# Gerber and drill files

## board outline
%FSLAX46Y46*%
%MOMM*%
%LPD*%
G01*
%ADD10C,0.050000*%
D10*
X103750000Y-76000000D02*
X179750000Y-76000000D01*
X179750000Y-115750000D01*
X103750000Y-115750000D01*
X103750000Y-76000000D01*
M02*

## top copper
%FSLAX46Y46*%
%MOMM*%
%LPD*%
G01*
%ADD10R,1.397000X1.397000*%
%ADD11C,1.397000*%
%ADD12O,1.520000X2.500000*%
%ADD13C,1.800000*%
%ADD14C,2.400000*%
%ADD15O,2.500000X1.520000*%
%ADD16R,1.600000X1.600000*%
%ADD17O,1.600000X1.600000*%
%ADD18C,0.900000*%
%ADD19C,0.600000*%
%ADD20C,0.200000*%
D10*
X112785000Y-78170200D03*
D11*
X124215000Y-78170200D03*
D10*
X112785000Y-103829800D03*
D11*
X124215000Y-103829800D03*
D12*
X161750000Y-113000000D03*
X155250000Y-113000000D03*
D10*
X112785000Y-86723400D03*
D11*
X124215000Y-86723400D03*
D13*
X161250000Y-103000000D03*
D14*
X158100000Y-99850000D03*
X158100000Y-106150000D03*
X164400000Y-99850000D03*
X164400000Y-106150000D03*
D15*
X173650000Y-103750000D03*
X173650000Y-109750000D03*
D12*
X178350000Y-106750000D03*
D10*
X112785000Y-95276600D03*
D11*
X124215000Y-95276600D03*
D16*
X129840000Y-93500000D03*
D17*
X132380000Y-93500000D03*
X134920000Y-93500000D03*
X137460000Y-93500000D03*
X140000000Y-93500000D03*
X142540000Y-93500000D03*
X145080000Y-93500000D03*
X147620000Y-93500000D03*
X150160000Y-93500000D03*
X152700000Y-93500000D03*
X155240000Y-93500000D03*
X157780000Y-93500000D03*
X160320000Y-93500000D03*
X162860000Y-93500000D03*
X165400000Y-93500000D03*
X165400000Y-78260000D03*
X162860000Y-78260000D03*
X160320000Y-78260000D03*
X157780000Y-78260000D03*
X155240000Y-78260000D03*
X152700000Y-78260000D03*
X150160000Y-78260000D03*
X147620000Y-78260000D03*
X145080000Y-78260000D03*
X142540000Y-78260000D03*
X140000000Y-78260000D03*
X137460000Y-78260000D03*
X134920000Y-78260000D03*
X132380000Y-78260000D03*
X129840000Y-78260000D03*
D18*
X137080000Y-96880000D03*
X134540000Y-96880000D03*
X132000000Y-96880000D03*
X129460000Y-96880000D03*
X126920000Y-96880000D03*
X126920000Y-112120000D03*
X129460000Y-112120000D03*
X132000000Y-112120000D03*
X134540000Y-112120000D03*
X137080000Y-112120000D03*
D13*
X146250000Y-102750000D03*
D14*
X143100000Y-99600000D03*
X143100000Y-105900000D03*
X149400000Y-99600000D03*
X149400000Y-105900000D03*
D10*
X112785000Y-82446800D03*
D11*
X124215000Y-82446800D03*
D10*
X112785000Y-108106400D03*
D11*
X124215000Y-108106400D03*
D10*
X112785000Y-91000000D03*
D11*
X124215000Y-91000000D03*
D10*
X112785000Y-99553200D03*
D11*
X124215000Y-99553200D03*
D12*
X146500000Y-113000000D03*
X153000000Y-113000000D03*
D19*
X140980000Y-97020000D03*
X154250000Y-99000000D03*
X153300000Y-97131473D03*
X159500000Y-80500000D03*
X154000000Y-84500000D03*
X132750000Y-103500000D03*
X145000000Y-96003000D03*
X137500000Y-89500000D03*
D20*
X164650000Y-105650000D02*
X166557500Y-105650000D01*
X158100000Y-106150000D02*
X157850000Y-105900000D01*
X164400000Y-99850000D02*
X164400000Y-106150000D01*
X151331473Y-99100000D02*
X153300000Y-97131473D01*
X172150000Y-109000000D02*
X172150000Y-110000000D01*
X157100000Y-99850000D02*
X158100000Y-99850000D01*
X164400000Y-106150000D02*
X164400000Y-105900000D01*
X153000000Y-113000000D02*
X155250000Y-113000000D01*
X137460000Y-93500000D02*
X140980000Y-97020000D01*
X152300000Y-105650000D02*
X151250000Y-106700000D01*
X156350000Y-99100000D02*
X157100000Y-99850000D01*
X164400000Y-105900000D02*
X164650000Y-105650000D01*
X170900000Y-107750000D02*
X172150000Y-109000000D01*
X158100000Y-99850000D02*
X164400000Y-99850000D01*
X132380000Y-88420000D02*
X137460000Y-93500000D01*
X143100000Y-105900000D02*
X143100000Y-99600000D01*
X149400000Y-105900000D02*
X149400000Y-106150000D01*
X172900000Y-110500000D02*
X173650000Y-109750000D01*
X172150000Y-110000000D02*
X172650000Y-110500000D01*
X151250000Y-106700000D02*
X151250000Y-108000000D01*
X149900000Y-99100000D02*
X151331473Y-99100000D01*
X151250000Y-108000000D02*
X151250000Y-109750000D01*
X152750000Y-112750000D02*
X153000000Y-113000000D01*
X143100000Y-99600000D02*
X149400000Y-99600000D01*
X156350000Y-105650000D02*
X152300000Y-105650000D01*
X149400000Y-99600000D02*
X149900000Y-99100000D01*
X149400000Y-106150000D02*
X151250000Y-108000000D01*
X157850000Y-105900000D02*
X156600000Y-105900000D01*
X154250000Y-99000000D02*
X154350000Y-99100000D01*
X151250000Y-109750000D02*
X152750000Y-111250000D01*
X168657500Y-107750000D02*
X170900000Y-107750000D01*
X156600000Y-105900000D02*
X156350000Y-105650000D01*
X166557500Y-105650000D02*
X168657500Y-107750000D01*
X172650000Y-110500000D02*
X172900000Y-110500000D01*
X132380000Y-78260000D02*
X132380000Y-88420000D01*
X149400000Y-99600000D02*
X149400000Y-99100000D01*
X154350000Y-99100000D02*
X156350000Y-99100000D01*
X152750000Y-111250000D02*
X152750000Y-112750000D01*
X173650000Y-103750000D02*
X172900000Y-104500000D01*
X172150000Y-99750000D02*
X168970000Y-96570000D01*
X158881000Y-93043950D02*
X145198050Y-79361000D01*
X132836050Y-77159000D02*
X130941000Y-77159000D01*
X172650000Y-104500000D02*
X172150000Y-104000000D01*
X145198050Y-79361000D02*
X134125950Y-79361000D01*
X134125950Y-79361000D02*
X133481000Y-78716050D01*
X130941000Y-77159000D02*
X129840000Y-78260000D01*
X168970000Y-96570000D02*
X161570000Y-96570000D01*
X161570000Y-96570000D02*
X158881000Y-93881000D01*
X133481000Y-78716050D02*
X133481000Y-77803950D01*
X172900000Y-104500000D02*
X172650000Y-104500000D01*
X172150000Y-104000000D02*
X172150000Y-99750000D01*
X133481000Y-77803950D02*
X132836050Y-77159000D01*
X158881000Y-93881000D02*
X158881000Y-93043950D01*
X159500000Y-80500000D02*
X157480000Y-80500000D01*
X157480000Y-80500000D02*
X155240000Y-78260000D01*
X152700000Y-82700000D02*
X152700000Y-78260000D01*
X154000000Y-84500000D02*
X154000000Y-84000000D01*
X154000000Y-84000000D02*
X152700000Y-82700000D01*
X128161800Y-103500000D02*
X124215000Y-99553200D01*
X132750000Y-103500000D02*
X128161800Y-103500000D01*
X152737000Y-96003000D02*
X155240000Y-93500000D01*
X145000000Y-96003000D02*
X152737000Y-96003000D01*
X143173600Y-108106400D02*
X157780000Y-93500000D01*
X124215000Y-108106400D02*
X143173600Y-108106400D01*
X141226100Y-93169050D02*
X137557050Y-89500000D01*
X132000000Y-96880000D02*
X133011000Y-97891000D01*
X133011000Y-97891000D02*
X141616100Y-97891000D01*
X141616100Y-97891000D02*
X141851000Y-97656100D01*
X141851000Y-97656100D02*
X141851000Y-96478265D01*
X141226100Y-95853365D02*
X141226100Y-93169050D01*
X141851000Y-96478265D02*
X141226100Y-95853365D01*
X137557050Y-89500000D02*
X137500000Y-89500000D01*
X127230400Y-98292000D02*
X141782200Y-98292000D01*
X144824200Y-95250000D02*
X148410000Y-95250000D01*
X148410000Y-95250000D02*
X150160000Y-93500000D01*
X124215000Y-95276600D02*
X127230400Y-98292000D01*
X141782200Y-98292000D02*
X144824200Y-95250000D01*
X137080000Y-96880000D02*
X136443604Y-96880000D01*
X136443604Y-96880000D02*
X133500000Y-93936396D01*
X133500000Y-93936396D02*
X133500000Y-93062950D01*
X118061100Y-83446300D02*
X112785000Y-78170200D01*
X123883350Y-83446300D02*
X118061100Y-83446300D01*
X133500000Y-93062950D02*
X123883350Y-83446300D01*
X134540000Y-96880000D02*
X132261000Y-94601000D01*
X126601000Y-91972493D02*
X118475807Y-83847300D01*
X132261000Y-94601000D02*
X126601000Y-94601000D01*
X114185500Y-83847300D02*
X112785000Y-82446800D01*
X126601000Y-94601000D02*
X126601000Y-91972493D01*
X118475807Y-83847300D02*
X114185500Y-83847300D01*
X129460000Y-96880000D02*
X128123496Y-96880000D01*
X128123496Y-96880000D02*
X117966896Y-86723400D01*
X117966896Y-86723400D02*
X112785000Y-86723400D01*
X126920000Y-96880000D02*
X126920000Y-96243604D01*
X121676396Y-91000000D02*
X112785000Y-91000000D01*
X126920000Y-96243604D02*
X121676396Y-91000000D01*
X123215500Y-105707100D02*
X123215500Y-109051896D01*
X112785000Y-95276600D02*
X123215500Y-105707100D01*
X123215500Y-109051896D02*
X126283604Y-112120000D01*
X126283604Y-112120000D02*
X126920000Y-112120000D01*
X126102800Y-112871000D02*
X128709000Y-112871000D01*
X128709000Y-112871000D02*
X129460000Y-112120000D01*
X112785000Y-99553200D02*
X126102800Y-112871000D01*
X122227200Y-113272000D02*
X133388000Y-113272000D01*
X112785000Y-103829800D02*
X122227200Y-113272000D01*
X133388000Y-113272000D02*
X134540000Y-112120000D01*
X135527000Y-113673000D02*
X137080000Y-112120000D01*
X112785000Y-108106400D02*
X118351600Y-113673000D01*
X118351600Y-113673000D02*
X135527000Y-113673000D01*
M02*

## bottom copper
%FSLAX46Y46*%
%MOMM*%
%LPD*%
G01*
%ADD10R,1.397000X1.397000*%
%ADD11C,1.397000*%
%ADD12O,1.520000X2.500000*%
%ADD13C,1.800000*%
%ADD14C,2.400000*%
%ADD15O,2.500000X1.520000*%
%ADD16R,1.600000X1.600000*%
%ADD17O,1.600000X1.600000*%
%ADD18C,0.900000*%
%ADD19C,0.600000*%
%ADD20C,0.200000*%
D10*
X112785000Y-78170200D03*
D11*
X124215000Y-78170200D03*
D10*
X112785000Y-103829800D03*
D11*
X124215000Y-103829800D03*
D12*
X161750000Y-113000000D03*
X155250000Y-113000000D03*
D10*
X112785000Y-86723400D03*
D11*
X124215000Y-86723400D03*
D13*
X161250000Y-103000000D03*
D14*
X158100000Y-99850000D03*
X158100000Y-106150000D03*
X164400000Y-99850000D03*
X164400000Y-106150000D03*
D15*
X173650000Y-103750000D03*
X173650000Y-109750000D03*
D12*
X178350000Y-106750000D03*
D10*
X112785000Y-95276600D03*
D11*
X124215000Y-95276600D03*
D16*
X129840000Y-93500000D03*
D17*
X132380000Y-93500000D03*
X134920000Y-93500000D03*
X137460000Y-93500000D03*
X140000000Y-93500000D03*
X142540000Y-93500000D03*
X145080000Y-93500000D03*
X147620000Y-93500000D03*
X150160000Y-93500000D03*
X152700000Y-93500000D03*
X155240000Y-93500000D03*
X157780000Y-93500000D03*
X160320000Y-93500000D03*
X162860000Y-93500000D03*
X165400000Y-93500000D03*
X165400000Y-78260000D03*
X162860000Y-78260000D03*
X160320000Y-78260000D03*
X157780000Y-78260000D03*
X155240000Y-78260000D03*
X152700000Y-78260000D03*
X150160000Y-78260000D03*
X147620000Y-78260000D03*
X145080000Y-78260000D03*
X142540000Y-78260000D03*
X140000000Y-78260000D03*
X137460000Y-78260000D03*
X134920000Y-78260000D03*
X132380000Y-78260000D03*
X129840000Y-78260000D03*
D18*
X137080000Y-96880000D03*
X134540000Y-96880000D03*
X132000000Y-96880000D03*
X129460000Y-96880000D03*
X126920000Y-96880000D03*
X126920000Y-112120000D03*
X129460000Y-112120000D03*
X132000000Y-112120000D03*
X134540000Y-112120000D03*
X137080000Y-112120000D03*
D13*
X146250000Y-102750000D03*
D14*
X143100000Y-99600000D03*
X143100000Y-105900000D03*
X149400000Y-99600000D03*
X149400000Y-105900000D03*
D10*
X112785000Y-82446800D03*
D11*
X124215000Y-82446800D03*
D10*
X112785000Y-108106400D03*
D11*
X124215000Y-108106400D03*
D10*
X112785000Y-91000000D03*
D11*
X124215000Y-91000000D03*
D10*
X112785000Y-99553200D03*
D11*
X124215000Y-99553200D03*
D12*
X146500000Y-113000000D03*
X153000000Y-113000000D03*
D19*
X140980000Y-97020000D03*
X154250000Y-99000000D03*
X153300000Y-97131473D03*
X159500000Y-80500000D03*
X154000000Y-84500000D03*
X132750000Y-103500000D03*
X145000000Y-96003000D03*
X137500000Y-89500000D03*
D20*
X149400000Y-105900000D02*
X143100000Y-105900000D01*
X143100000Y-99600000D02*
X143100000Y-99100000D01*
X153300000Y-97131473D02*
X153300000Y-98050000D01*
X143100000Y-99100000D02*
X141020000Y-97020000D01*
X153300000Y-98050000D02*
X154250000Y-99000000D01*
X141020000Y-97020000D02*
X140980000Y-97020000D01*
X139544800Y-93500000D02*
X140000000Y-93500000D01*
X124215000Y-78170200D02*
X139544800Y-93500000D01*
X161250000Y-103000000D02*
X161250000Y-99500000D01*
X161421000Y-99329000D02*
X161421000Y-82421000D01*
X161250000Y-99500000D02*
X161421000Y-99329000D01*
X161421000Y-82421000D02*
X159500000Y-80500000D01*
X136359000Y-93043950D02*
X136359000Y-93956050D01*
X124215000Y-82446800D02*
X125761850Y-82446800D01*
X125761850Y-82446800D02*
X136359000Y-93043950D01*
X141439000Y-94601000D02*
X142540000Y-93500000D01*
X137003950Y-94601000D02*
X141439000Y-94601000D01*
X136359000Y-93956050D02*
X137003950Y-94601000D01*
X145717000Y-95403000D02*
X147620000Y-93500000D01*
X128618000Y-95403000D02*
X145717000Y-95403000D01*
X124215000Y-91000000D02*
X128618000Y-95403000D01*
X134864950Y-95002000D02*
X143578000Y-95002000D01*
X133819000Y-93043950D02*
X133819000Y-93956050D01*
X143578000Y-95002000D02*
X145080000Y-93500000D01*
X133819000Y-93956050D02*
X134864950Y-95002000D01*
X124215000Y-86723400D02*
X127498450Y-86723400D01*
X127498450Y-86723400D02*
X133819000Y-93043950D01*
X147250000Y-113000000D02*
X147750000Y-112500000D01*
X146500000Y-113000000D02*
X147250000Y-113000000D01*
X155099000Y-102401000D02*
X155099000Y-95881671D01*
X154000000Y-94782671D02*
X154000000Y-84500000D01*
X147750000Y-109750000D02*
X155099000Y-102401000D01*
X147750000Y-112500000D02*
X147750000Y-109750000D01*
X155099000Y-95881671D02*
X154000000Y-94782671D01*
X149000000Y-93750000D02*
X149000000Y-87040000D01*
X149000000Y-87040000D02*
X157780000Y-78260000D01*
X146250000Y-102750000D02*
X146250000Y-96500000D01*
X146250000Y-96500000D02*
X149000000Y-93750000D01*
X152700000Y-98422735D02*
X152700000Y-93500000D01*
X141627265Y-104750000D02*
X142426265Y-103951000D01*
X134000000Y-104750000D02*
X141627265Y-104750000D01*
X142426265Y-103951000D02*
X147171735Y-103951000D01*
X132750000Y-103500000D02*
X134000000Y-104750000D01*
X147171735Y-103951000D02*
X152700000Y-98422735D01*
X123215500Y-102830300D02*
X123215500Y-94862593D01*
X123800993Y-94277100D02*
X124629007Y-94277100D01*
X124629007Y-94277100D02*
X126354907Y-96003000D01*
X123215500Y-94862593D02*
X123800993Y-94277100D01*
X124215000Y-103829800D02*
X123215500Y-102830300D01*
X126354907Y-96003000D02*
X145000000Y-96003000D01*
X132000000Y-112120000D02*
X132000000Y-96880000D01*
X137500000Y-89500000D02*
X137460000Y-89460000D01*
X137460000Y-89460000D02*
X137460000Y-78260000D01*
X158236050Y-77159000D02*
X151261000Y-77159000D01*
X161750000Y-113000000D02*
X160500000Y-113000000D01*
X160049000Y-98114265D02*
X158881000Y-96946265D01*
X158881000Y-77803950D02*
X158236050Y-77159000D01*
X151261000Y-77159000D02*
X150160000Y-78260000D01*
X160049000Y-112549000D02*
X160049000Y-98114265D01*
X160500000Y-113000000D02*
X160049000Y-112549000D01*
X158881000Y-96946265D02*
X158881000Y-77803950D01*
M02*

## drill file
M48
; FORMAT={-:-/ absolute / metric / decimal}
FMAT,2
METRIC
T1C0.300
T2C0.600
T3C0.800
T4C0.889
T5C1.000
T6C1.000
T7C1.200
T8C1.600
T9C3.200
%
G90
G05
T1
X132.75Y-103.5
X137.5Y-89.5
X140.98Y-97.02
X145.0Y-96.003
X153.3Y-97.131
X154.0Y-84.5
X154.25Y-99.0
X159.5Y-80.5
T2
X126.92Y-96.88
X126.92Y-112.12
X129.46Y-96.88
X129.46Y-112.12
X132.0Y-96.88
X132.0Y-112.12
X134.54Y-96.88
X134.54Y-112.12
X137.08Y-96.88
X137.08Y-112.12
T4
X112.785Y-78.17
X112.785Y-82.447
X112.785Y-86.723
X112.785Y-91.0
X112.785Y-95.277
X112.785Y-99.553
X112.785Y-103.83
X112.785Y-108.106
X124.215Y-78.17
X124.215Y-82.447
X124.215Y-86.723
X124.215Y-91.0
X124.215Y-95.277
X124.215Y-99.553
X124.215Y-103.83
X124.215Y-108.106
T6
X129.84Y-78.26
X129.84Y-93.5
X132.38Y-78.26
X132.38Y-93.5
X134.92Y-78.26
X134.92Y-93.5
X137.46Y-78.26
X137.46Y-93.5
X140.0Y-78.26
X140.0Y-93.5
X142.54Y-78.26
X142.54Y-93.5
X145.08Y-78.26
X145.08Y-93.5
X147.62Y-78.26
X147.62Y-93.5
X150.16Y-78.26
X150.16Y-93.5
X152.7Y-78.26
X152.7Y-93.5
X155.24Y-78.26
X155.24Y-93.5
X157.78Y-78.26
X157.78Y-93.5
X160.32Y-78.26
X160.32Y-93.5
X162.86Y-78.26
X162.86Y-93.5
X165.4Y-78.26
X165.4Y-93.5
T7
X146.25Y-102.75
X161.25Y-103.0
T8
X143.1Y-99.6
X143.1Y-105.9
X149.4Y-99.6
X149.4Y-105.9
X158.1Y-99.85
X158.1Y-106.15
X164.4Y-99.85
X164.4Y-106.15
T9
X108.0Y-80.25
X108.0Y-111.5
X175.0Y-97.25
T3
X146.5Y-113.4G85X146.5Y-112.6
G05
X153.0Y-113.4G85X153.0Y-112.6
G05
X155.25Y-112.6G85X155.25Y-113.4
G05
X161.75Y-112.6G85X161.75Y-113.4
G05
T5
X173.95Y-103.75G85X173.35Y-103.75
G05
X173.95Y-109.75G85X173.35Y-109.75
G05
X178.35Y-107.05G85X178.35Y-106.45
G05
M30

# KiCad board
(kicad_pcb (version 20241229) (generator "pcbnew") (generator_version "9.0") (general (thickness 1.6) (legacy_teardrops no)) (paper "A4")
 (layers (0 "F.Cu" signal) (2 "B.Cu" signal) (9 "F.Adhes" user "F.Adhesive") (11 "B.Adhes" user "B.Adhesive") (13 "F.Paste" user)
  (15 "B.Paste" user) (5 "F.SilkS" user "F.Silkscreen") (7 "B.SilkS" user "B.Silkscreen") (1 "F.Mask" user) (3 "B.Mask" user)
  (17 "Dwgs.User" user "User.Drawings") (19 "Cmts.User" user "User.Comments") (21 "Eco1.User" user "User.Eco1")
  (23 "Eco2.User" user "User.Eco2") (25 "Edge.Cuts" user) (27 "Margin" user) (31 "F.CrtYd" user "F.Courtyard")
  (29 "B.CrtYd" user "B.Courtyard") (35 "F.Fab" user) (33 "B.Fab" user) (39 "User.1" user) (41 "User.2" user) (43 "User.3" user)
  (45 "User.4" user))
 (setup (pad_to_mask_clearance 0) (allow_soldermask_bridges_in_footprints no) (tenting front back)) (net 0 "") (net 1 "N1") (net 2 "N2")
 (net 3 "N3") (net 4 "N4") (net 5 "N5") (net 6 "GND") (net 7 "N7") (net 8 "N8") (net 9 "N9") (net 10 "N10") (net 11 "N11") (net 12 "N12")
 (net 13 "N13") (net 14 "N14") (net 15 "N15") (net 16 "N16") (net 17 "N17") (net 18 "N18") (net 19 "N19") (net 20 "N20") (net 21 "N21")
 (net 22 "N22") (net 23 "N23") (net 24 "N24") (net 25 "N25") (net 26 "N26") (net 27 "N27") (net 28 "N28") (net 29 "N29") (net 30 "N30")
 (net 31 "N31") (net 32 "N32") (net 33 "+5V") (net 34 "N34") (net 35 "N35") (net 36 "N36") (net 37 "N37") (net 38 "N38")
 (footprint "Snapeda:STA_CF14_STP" (layer "F.Cu") (at 112.785 78.1702)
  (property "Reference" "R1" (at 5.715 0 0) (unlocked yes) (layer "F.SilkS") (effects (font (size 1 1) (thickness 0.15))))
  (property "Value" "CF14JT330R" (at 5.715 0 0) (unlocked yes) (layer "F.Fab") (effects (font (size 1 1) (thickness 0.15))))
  (pad "1" thru_hole rect (at 0 0) (size 1.397 1.397) (drill 0.889) (layers "*.Cu" "*.Mask") (remove_unused_layers no) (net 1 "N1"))
  (pad "2" thru_hole circle (at 11.43 0) (size 1.397 1.397) (drill 0.889) (layers "*.Cu" "*.Mask") (remove_unused_layers no) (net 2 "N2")))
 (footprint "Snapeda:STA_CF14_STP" (layer "F.Cu") (at 112.785 103.8298)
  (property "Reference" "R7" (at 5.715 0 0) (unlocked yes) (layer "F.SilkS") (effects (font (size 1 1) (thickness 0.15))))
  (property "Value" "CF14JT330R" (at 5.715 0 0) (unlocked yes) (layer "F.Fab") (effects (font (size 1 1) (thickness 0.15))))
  (pad "1" thru_hole rect (at 0 0) (size 1.397 1.397) (drill 0.889) (layers "*.Cu" "*.Mask") (remove_unused_layers no) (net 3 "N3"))
  (pad "2" thru_hole circle (at 11.43 0) (size 1.397 1.397) (drill 0.889) (layers "*.Cu" "*.Mask") (remove_unused_layers no) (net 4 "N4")))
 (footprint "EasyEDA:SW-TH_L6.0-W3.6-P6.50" (layer "F.Cu") (at 158.5 113)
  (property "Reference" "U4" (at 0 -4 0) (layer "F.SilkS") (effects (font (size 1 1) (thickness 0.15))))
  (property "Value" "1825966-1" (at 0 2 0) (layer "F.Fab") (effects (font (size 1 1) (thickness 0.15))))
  (pad "1" thru_hole oval (at 3.25 0 270) (size 2.5 1.52) (drill oval 1.599997 0.799998) (layers "*.Cu" "*.Mask") (remove_unused_layers no)
   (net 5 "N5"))
  (pad "2" thru_hole oval (at -3.25 0 270) (size 2.5 1.52) (drill oval 1.599997 0.799998) (layers "*.Cu" "*.Mask") (remove_unused_layers no)
   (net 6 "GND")))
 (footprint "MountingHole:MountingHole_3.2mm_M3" (layer "F.Cu") (at 175 97.25)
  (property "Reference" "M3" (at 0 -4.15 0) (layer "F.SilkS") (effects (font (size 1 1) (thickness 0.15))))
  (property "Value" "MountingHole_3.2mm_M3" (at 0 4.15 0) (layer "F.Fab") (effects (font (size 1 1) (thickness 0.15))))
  (pad "" np_thru_hole circle (at 0 0) (size 3.2 3.2) (drill 3.2) (layers "*.Cu" "*.Mask")))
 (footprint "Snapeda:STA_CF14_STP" (layer "F.Cu") (at 112.785 86.7234)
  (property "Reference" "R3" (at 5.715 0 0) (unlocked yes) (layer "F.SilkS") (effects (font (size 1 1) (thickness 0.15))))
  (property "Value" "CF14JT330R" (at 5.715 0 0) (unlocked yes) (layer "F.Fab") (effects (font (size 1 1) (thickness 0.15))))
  (pad "1" thru_hole rect (at 0 0) (size 1.397 1.397) (drill 0.889) (layers "*.Cu" "*.Mask") (remove_unused_layers no) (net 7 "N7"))
  (pad "2" thru_hole circle (at 11.43 0) (size 1.397 1.397) (drill 0.889) (layers "*.Cu" "*.Mask") (remove_unused_layers no) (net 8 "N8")))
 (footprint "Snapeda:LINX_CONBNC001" (layer "F.Cu") (at 161.25 103)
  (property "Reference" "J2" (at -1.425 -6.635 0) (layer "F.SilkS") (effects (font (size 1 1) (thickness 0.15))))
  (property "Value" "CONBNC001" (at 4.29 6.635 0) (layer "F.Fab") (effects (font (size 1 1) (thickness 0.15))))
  (pad "1" thru_hole circle (at 0 0) (size 1.8 1.8) (drill 1.2) (layers "*.Cu" "*.Mask") (remove_unused_layers no) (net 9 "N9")
   (solder_mask_margin 0.102))
  (pad "S1" thru_hole circle (at -3.15 -3.15) (size 2.4 2.4) (drill 1.6) (layers "*.Cu" "*.Mask") (remove_unused_layers no) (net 6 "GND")
   (solder_mask_margin 0.102))
  (pad "S1" thru_hole circle (at -3.15 3.15) (size 2.4 2.4) (drill 1.6) (layers "*.Cu" "*.Mask") (remove_unused_layers no) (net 6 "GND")
   (solder_mask_margin 0.102))
  (pad "S1" thru_hole circle (at 3.15 -3.15) (size 2.4 2.4) (drill 1.6) (layers "*.Cu" "*.Mask") (remove_unused_layers no) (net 6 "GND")
   (solder_mask_margin 0.102))
  (pad "S1" thru_hole circle (at 3.15 3.15) (size 2.4 2.4) (drill 1.6) (layers "*.Cu" "*.Mask") (remove_unused_layers no) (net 6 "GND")
   (solder_mask_margin 0.102)))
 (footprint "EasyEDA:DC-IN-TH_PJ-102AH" (layer "F.Cu") (at 176 106.75 180)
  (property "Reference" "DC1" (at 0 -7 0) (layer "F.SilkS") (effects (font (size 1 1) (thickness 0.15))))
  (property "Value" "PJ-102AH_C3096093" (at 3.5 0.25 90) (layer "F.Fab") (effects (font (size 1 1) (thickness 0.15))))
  (pad "1" thru_hole oval (at 2.35 3 180) (size 2.5 1.52) (drill oval 1.599997 0.999998) (layers "*.Cu" "*.Mask") (remove_unused_layers no)
   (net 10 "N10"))
  (pad "2" thru_hole oval (at 2.35 -3 180) (size 2.5 1.52) (drill oval 1.599997 0.999998) (layers "*.Cu" "*.Mask") (remove_unused_layers no)
   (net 6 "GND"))
  (pad "3" thru_hole oval (at -2.35 0 90) (size 2.5 1.52) (drill oval 1.599997 0.999998) (layers "*.Cu" "*.Mask") (remove_unused_layers no)
   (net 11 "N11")))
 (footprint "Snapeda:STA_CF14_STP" (layer "F.Cu") (at 112.785 95.2766)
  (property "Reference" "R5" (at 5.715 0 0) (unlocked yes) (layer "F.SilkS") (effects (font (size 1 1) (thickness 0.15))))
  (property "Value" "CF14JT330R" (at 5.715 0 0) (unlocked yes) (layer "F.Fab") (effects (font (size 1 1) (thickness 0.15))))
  (pad "1" thru_hole rect (at 0 0) (size 1.397 1.397) (drill 0.889) (layers "*.Cu" "*.Mask") (remove_unused_layers no) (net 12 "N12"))
  (pad "2" thru_hole circle (at 11.43 0) (size 1.397 1.397) (drill 0.889) (layers "*.Cu" "*.Mask") (remove_unused_layers no) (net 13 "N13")))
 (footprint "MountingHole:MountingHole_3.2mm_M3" (layer "F.Cu") (at 108 111.5)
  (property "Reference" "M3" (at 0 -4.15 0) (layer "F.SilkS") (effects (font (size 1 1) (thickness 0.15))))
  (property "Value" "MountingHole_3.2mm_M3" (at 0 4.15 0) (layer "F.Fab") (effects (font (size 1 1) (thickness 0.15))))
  (pad "" np_thru_hole circle (at 0 0) (size 3.2 3.2) (drill 3.2) (layers "*.Cu" "*.Mask")))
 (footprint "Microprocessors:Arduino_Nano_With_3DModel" (layer "F.Cu") (at 129.84 93.5 90)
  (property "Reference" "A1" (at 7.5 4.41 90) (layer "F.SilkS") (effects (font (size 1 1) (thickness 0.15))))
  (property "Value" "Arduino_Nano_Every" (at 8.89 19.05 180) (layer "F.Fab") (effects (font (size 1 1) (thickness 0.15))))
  (pad "1" thru_hole rect (at 0 0 90) (size 1.6 1.6) (drill 1) (layers "*.Cu" "*.Mask") (remove_unused_layers no) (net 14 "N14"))
  (pad "2" thru_hole oval (at 0 2.54 90) (size 1.6 1.6) (drill 1) (layers "*.Cu" "*.Mask") (remove_unused_layers no) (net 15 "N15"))
  (pad "3" thru_hole oval (at 0 5.08 90) (size 1.6 1.6) (drill 1) (layers "*.Cu" "*.Mask") (remove_unused_layers no) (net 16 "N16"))
  (pad "4" thru_hole oval (at 0 7.62 90) (size 1.6 1.6) (drill 1) (layers "*.Cu" "*.Mask") (remove_unused_layers no) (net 6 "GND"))
  (pad "5" thru_hole oval (at 0 10.16 90) (size 1.6 1.6) (drill 1) (layers "*.Cu" "*.Mask") (remove_unused_layers no) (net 2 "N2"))
  (pad "6" thru_hole oval (at 0 12.7 90) (size 1.6 1.6) (drill 1) (layers "*.Cu" "*.Mask") (remove_unused_layers no) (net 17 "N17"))
  (pad "7" thru_hole oval (at 0 15.24 90) (size 1.6 1.6) (drill 1) (layers "*.Cu" "*.Mask") (remove_unused_layers no) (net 8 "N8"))
  (pad "8" thru_hole oval (at 0 17.78 90) (size 1.6 1.6) (drill 1) (layers "*.Cu" "*.Mask") (remove_unused_layers no) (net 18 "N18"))
  (pad "9" thru_hole oval (at 0 20.32 90) (size 1.6 1.6) (drill 1) (layers "*.Cu" "*.Mask") (remove_unused_layers no) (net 13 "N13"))
  (pad "10" thru_hole oval (at 0 22.86 90) (size 1.6 1.6) (drill 1) (layers "*.Cu" "*.Mask") (remove_unused_layers no) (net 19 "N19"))
  (pad "11" thru_hole oval (at 0 25.4 90) (size 1.6 1.6) (drill 1) (layers "*.Cu" "*.Mask") (remove_unused_layers no) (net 4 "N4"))
  (pad "12" thru_hole oval (at 0 27.94 90) (size 1.6 1.6) (drill 1) (layers "*.Cu" "*.Mask") (remove_unused_layers no) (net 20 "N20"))
  (pad "13" thru_hole oval (at 0 30.48 90) (size 1.6 1.6) (drill 1) (layers "*.Cu" "*.Mask") (remove_unused_layers no) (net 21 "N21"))
  (pad "14" thru_hole oval (at 0 33.02 90) (size 1.6 1.6) (drill 1) (layers "*.Cu" "*.Mask") (remove_unused_layers no) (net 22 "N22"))
  (pad "15" thru_hole oval (at 0 35.56 90) (size 1.6 1.6) (drill 1) (layers "*.Cu" "*.Mask") (remove_unused_layers no) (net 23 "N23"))
  (pad "16" thru_hole oval (at 15.24 35.56 90) (size 1.6 1.6) (drill 1) (layers "*.Cu" "*.Mask") (remove_unused_layers no) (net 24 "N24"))
  (pad "17" thru_hole oval (at 15.24 33.02 90) (size 1.6 1.6) (drill 1) (layers "*.Cu" "*.Mask") (remove_unused_layers no) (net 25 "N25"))
  (pad "18" thru_hole oval (at 15.24 30.48 90) (size 1.6 1.6) (drill 1) (layers "*.Cu" "*.Mask") (remove_unused_layers no) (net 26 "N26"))
  (pad "19" thru_hole oval (at 15.24 27.94 90) (size 1.6 1.6) (drill 1) (layers "*.Cu" "*.Mask") (remove_unused_layers no) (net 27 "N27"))
  (pad "20" thru_hole oval (at 15.24 25.4 90) (size 1.6 1.6) (drill 1) (layers "*.Cu" "*.Mask") (remove_unused_layers no) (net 9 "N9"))
  (pad "21" thru_hole oval (at 15.24 22.86 90) (size 1.6 1.6) (drill 1) (layers "*.Cu" "*.Mask") (remove_unused_layers no) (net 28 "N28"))
  (pad "22" thru_hole oval (at 15.24 20.32 90) (size 1.6 1.6) (drill 1) (layers "*.Cu" "*.Mask") (remove_unused_layers no) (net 5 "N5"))
  (pad "23" thru_hole oval (at 15.24 17.78 90) (size 1.6 1.6) (drill 1) (layers "*.Cu" "*.Mask") (remove_unused_layers no) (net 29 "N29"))
  (pad "24" thru_hole oval (at 15.24 15.24 90) (size 1.6 1.6) (drill 1) (layers "*.Cu" "*.Mask") (remove_unused_layers no) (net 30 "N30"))
  (pad "25" thru_hole oval (at 15.24 12.7 90) (size 1.6 1.6) (drill 1) (layers "*.Cu" "*.Mask") (remove_unused_layers no) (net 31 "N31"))
  (pad "26" thru_hole oval (at 15.24 10.16 90) (size 1.6 1.6) (drill 1) (layers "*.Cu" "*.Mask") (remove_unused_layers no) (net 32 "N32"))
  (pad "27" thru_hole oval (at 15.24 7.62 90) (size 1.6 1.6) (drill 1) (layers "*.Cu" "*.Mask") (remove_unused_layers no) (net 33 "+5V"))
  (pad "28" thru_hole oval (at 15.24 5.08 90) (size 1.6 1.6) (drill 1) (layers "*.Cu" "*.Mask") (remove_unused_layers no) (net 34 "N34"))
  (pad "29" thru_hole oval (at 15.24 2.54 90) (size 1.6 1.6) (drill 1) (layers "*.Cu" "*.Mask") (remove_unused_layers no) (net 6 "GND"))
  (pad "30" thru_hole oval (at 15.24 0 90) (size 1.6 1.6) (drill 1) (layers "*.Cu" "*.Mask") (remove_unused_layers no) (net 10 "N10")))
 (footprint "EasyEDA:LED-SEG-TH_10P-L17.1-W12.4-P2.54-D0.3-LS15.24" (layer "F.Cu") (at 132 104.5 180)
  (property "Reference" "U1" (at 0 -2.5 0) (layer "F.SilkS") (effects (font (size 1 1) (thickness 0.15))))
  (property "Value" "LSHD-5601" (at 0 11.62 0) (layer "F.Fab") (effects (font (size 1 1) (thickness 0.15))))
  (pad "1" thru_hole circle (at -5.08 7.62 180) (size 0.9 0.9) (drill 0.599999) (layers "*.Cu" "*.Mask") (remove_unused_layers no)
   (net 1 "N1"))
  (pad "2" thru_hole circle (at -2.54 7.62 180) (size 0.9 0.9) (drill 0.599999) (layers "*.Cu" "*.Mask") (remove_unused_layers no)
   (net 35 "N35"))
  (pad "3" thru_hole circle (at 0 7.62 180) (size 0.9 0.9) (drill 0.599999) (layers "*.Cu" "*.Mask") (remove_unused_layers no)
   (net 33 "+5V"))
  (pad "4" thru_hole circle (at 2.54 7.62 180) (size 0.9 0.9) (drill 0.599999) (layers "*.Cu" "*.Mask") (remove_unused_layers no)
   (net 7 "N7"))
  (pad "5" thru_hole circle (at 5.08 7.62 180) (size 0.9 0.9) (drill 0.599999) (layers "*.Cu" "*.Mask") (remove_unused_layers no)
   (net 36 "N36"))
  (pad "6" thru_hole circle (at 5.08 -7.62 180) (size 0.9 0.9) (drill 0.599999) (layers "*.Cu" "*.Mask") (remove_unused_layers no)
   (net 12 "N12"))
  (pad "7" thru_hole circle (at 2.54 -7.62 180) (size 0.9 0.9) (drill 0.599999) (layers "*.Cu" "*.Mask") (remove_unused_layers no)
   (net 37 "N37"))
  (pad "8" thru_hole circle (at 0 -7.62 180) (size 0.9 0.9) (drill 0.599999) (layers "*.Cu" "*.Mask") (remove_unused_layers no)
   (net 33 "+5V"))
  (pad "9" thru_hole circle (at -2.54 -7.62 180) (size 0.9 0.9) (drill 0.599999) (layers "*.Cu" "*.Mask") (remove_unused_layers no)
   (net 3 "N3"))
  (pad "10" thru_hole circle (at -5.08 -7.62 180) (size 0.9 0.9) (drill 0.599999) (layers "*.Cu" "*.Mask") (remove_unused_layers no)
   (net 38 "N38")))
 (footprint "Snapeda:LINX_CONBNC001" (layer "F.Cu") (at 146.25 102.75)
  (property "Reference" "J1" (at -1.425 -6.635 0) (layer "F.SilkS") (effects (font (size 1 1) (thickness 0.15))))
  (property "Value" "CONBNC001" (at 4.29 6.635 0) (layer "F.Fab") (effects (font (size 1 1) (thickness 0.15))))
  (pad "1" thru_hole circle (at 0 0) (size 1.8 1.8) (drill 1.2) (layers "*.Cu" "*.Mask") (remove_unused_layers no) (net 27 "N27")
   (solder_mask_margin 0.102))
  (pad "S1" thru_hole circle (at -3.15 -3.15) (size 2.4 2.4) (drill 1.6) (layers "*.Cu" "*.Mask") (remove_unused_layers no) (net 6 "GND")
   (solder_mask_margin 0.102))
  (pad "S1" thru_hole circle (at -3.15 3.15) (size 2.4 2.4) (drill 1.6) (layers "*.Cu" "*.Mask") (remove_unused_layers no) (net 6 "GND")
   (solder_mask_margin 0.102))
  (pad "S1" thru_hole circle (at 3.15 -3.15) (size 2.4 2.4) (drill 1.6) (layers "*.Cu" "*.Mask") (remove_unused_layers no) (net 6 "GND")
   (solder_mask_margin 0.102))
  (pad "S1" thru_hole circle (at 3.15 3.15) (size 2.4 2.4) (drill 1.6) (layers "*.Cu" "*.Mask") (remove_unused_layers no) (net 6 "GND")
   (solder_mask_margin 0.102)))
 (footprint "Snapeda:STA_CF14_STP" (layer "F.Cu") (at 112.785 82.4468)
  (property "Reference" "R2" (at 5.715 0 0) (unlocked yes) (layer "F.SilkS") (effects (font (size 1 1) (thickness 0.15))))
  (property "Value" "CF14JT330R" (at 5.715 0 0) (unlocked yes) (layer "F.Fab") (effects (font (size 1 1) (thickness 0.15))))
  (pad "1" thru_hole rect (at 0 0) (size 1.397 1.397) (drill 0.889) (layers "*.Cu" "*.Mask") (remove_unused_layers no) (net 35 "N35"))
  (pad "2" thru_hole circle (at 11.43 0) (size 1.397 1.397) (drill 0.889) (layers "*.Cu" "*.Mask") (remove_unused_layers no) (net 17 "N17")))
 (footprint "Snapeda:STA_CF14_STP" (layer "F.Cu") (at 112.785 108.1064)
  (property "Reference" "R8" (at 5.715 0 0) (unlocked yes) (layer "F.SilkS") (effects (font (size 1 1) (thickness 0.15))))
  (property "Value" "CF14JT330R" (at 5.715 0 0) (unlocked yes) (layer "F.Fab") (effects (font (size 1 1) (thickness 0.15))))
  (pad "1" thru_hole rect (at 0 0) (size 1.397 1.397) (drill 0.889) (layers "*.Cu" "*.Mask") (remove_unused_layers no) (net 38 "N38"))
  (pad "2" thru_hole circle (at 11.43 0) (size 1.397 1.397) (drill 0.889) (layers "*.Cu" "*.Mask") (remove_unused_layers no) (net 20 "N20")))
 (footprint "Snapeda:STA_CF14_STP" (layer "F.Cu") (at 112.785 91)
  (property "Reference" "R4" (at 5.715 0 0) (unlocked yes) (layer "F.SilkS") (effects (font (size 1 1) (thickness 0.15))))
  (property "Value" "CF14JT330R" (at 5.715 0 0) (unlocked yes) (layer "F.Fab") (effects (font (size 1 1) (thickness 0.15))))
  (pad "1" thru_hole rect (at 0 0) (size 1.397 1.397) (drill 0.889) (layers "*.Cu" "*.Mask") (remove_unused_layers no) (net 36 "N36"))
  (pad "2" thru_hole circle (at 11.43 0) (size 1.397 1.397) (drill 0.889) (layers "*.Cu" "*.Mask") (remove_unused_layers no) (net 18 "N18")))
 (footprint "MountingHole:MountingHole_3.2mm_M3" (layer "F.Cu") (at 108 80.25)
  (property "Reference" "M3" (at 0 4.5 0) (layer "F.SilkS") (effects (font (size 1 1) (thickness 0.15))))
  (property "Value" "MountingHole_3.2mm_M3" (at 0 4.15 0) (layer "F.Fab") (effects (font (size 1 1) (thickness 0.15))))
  (pad "" np_thru_hole circle (at 0 0) (size 3.2 3.2) (drill 3.2) (layers "*.Cu" "*.Mask")))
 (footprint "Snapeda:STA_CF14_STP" (layer "F.Cu") (at 112.785 99.5532)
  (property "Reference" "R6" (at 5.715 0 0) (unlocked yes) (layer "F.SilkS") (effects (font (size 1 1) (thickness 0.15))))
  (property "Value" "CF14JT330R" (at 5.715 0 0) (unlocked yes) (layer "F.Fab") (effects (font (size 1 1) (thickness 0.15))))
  (pad "1" thru_hole rect (at 0 0) (size 1.397 1.397) (drill 0.889) (layers "*.Cu" "*.Mask") (remove_unused_layers no) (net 37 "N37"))
  (pad "2" thru_hole circle (at 11.43 0) (size 1.397 1.397) (drill 0.889) (layers "*.Cu" "*.Mask") (remove_unused_layers no) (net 19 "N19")))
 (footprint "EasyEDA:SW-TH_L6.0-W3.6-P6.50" (layer "F.Cu") (at 149.75 113 180)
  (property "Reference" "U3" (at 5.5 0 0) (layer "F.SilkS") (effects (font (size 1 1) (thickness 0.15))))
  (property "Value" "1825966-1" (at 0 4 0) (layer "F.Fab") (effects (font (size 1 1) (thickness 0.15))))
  (pad "1" thru_hole oval (at 3.25 0 90) (size 2.5 1.52) (drill oval 1.599997 0.799998) (layers "*.Cu" "*.Mask") (remove_unused_layers no)
   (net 28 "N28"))
  (pad "2" thru_hole oval (at -3.25 0 90) (size 2.5 1.52) (drill oval 1.599997 0.799998) (layers "*.Cu" "*.Mask") (remove_unused_layers no)
   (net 6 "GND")))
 (gr_rect (start 103.75 76) (end 179.75 115.75) (stroke (width 0.05) (type default)) (fill no) (layer "Edge.Cuts"))
 (segment (start 164.65 105.65) (end 166.5575 105.65) (width 0.2) (layer "F.Cu") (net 6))
 (segment (start 158.1 106.15) (end 157.85 105.9) (width 0.2) (layer "F.Cu") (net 6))
 (segment (start 164.4 99.85) (end 164.4 106.15) (width 0.2) (layer "F.Cu") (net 6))
 (segment (start 151.331473 99.1) (end 153.3 97.131473) (width 0.2) (layer "F.Cu") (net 6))
 (segment (start 172.15 109) (end 172.15 110) (width 0.2) (layer "F.Cu") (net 6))
 (segment (start 157.1 99.85) (end 158.1 99.85) (width 0.2) (layer "F.Cu") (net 6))
 (segment (start 164.4 106.15) (end 164.4 105.9) (width 0.2) (layer "F.Cu") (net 6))
 (segment (start 153 113) (end 155.25 113) (width 0.2) (layer "F.Cu") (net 6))
 (segment (start 137.46 93.5) (end 140.98 97.02) (width 0.2) (layer "F.Cu") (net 6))
 (segment (start 152.3 105.65) (end 151.25 106.7) (width 0.2) (layer "F.Cu") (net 6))
 (segment (start 156.35 99.1) (end 157.1 99.85) (width 0.2) (layer "F.Cu") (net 6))
 (segment (start 164.4 105.9) (end 164.65 105.65) (width 0.2) (layer "F.Cu") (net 6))
 (segment (start 170.9 107.75) (end 172.15 109) (width 0.2) (layer "F.Cu") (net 6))
 (segment (start 158.1 99.85) (end 164.4 99.85) (width 0.2) (layer "F.Cu") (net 6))
 (segment (start 132.38 88.42) (end 137.46 93.5) (width 0.2) (layer "F.Cu") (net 6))
 (segment (start 143.1 105.9) (end 143.1 99.6) (width 0.2) (layer "F.Cu") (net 6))
 (segment (start 149.4 105.9) (end 149.4 106.15) (width 0.2) (layer "F.Cu") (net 6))
 (segment (start 172.9 110.5) (end 173.65 109.75) (width 0.2) (layer "F.Cu") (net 6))
 (segment (start 172.15 110) (end 172.65 110.5) (width 0.2) (layer "F.Cu") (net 6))
 (segment (start 151.25 106.7) (end 151.25 108) (width 0.2) (layer "F.Cu") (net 6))
 (segment (start 149.9 99.1) (end 151.331473 99.1) (width 0.2) (layer "F.Cu") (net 6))
 (segment (start 151.25 108) (end 151.25 109.75) (width 0.2) (layer "F.Cu") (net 6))
 (segment (start 152.75 112.75) (end 153 113) (width 0.2) (layer "F.Cu") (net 6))
 (segment (start 143.1 99.6) (end 149.4 99.6) (width 0.2) (layer "F.Cu") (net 6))
 (segment (start 156.35 105.65) (end 152.3 105.65) (width 0.2) (layer "F.Cu") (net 6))
 (segment (start 149.4 99.6) (end 149.9 99.1) (width 0.2) (layer "F.Cu") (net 6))
 (segment (start 149.4 106.15) (end 151.25 108) (width 0.2) (layer "F.Cu") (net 6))
 (segment (start 157.85 105.9) (end 156.6 105.9) (width 0.2) (layer "F.Cu") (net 6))
 (segment (start 154.25 99) (end 154.35 99.1) (width 0.2) (layer "F.Cu") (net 6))
 (segment (start 151.25 109.75) (end 152.75 111.25) (width 0.2) (layer "F.Cu") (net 6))
 (segment (start 168.6575 107.75) (end 170.9 107.75) (width 0.2) (layer "F.Cu") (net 6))
 (segment (start 156.6 105.9) (end 156.35 105.65) (width 0.2) (layer "F.Cu") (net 6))
 (segment (start 166.5575 105.65) (end 168.6575 107.75) (width 0.2) (layer "F.Cu") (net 6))
 (segment (start 172.65 110.5) (end 172.9 110.5) (width 0.2) (layer "F.Cu") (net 6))
 (segment (start 132.38 78.26) (end 132.38 88.42) (width 0.2) (layer "F.Cu") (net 6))
 (segment (start 149.4 99.6) (end 149.4 99.1) (width 0.2) (layer "F.Cu") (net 6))
 (segment (start 154.35 99.1) (end 156.35 99.1) (width 0.2) (layer "F.Cu") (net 6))
 (segment (start 152.75 111.25) (end 152.75 112.75) (width 0.2) (layer "F.Cu") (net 6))
 (via (at 140.98 97.02) (size 0.6) (drill 0.3) (layers "F.Cu" "B.Cu") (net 6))
 (via (at 154.25 99) (size 0.6) (drill 0.3) (layers "F.Cu" "B.Cu") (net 6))
 (via (at 153.3 97.131473) (size 0.6) (drill 0.3) (layers "F.Cu" "B.Cu") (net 6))
 (segment (start 149.4 105.9) (end 143.1 105.9) (width 0.2) (layer "B.Cu") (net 6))
 (segment (start 143.1 99.6) (end 143.1 99.1) (width 0.2) (layer "B.Cu") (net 6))
 (segment (start 153.3 97.131473) (end 153.3 98.05) (width 0.2) (layer "B.Cu") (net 6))
 (segment (start 143.1 99.1) (end 141.02 97.02) (width 0.2) (layer "B.Cu") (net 6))
 (segment (start 153.3 98.05) (end 154.25 99) (width 0.2) (layer "B.Cu") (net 6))
 (segment (start 141.02 97.02) (end 140.98 97.02) (width 0.2) (layer "B.Cu") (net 6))
 (segment (start 173.65 103.75) (end 172.9 104.5) (width 0.2) (layer "F.Cu") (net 10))
 (segment (start 172.15 99.75) (end 168.97 96.57) (width 0.2) (layer "F.Cu") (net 10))
 (segment (start 158.881 93.04395) (end 145.19805 79.361) (width 0.2) (layer "F.Cu") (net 10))
 (segment (start 132.83605 77.159) (end 130.941 77.159) (width 0.2) (layer "F.Cu") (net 10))
 (segment (start 172.65 104.5) (end 172.15 104) (width 0.2) (layer "F.Cu") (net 10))
 (segment (start 145.19805 79.361) (end 134.12595 79.361) (width 0.2) (layer "F.Cu") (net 10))
 (segment (start 134.12595 79.361) (end 133.481 78.71605) (width 0.2) (layer "F.Cu") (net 10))
 (segment (start 130.941 77.159) (end 129.84 78.26) (width 0.2) (layer "F.Cu") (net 10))
 (segment (start 168.97 96.57) (end 161.57 96.57) (width 0.2) (layer "F.Cu") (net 10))
 (segment (start 161.57 96.57) (end 158.881 93.881) (width 0.2) (layer "F.Cu") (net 10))
 (segment (start 133.481 78.71605) (end 133.481 77.80395) (width 0.2) (layer "F.Cu") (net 10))
 (segment (start 172.9 104.5) (end 172.65 104.5) (width 0.2) (layer "F.Cu") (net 10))
 (segment (start 172.15 104) (end 172.15 99.75) (width 0.2) (layer "F.Cu") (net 10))
 (segment (start 133.481 77.80395) (end 132.83605 77.159) (width 0.2) (layer "F.Cu") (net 10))
 (segment (start 158.881 93.881) (end 158.881 93.04395) (width 0.2) (layer "F.Cu") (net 10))
 (segment (start 139.5448 93.5) (end 140 93.5) (width 0.2) (layer "B.Cu") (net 2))
 (segment (start 124.215 78.1702) (end 139.5448 93.5) (width 0.2) (layer "B.Cu") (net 2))
 (segment (start 159.5 80.5) (end 157.48 80.5) (width 0.2) (layer "F.Cu") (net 9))
 (segment (start 157.48 80.5) (end 155.24 78.26) (width 0.2) (layer "F.Cu") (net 9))
 (via (at 159.5 80.5) (size 0.6) (drill 0.3) (layers "F.Cu" "B.Cu") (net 9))
 (segment (start 161.25 103) (end 161.25 99.5) (width 0.2) (layer "B.Cu") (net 9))
 (segment (start 161.421 99.329) (end 161.421 82.421) (width 0.2) (layer "B.Cu") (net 9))
 (segment (start 161.25 99.5) (end 161.421 99.329) (width 0.2) (layer "B.Cu") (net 9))
 (segment (start 161.421 82.421) (end 159.5 80.5) (width 0.2) (layer "B.Cu") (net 9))
 (segment (start 136.359 93.04395) (end 136.359 93.95605) (width 0.2) (layer "B.Cu") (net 17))
 (segment (start 124.215 82.4468) (end 125.76185 82.4468) (width 0.2) (layer "B.Cu") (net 17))
 (segment (start 125.76185 82.4468) (end 136.359 93.04395) (width 0.2) (layer "B.Cu") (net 17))
 (segment (start 141.439 94.601) (end 142.54 93.5) (width 0.2) (layer "B.Cu") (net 17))
 (segment (start 137.00395 94.601) (end 141.439 94.601) (width 0.2) (layer "B.Cu") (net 17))
 (segment (start 136.359 93.95605) (end 137.00395 94.601) (width 0.2) (layer "B.Cu") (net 17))
 (segment (start 145.717 95.403) (end 147.62 93.5) (width 0.2) (layer "B.Cu") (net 18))
 (segment (start 128.618 95.403) (end 145.717 95.403) (width 0.2) (layer "B.Cu") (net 18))
 (segment (start 124.215 91) (end 128.618 95.403) (width 0.2) (layer "B.Cu") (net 18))
 (segment (start 134.86495 95.002) (end 143.578 95.002) (width 0.2) (layer "B.Cu") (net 8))
 (segment (start 133.819 93.04395) (end 133.819 93.95605) (width 0.2) (layer "B.Cu") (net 8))
 (segment (start 143.578 95.002) (end 145.08 93.5) (width 0.2) (layer "B.Cu") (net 8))
 (segment (start 133.819 93.95605) (end 134.86495 95.002) (width 0.2) (layer "B.Cu") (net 8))
 (segment (start 124.215 86.7234) (end 127.49845 86.7234) (width 0.2) (layer "B.Cu") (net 8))
 (segment (start 127.49845 86.7234) (end 133.819 93.04395) (width 0.2) (layer "B.Cu") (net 8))
 (segment (start 152.7 82.7) (end 152.7 78.26) (width 0.2) (layer "F.Cu") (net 28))
 (segment (start 154 84.5) (end 154 84) (width 0.2) (layer "F.Cu") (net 28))
 (segment (start 154 84) (end 152.7 82.7) (width 0.2) (layer "F.Cu") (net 28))
 (via (at 154 84.5) (size 0.6) (drill 0.3) (layers "F.Cu" "B.Cu") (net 28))
 (segment (start 147.25 113) (end 147.75 112.5) (width 0.2) (layer "B.Cu") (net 28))
 (segment (start 146.5 113) (end 147.25 113) (width 0.2) (layer "B.Cu") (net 28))
 (segment (start 155.099 102.401) (end 155.099 95.881671) (width 0.2) (layer "B.Cu") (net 28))
 (segment (start 154 94.782671) (end 154 84.5) (width 0.2) (layer "B.Cu") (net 28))
 (segment (start 147.75 109.75) (end 155.099 102.401) (width 0.2) (layer "B.Cu") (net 28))
 (segment (start 147.75 112.5) (end 147.75 109.75) (width 0.2) (layer "B.Cu") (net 28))
 (segment (start 155.099 95.881671) (end 154 94.782671) (width 0.2) (layer "B.Cu") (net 28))
 (segment (start 149 93.75) (end 149 87.04) (width 0.2) (layer "B.Cu") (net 27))
 (segment (start 149 87.04) (end 157.78 78.26) (width 0.2) (layer "B.Cu") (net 27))
 (segment (start 146.25 102.75) (end 146.25 96.5) (width 0.2) (layer "B.Cu") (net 27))
 (segment (start 146.25 96.5) (end 149 93.75) (width 0.2) (layer "B.Cu") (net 27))
 (segment (start 128.1618 103.5) (end 124.215 99.5532) (width 0.2) (layer "F.Cu") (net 19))
 (segment (start 132.75 103.5) (end 128.1618 103.5) (width 0.2) (layer "F.Cu") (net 19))
 (via (at 132.75 103.5) (size 0.6) (drill 0.3) (layers "F.Cu" "B.Cu") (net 19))
 (segment (start 152.7 98.422735) (end 152.7 93.5) (width 0.2) (layer "B.Cu") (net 19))
 (segment (start 141.627265 104.75) (end 142.426265 103.951) (width 0.2) (layer "B.Cu") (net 19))
 (segment (start 134 104.75) (end 141.627265 104.75) (width 0.2) (layer "B.Cu") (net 19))
 (segment (start 142.426265 103.951) (end 147.171735 103.951) (width 0.2) (layer "B.Cu") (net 19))
 (segment (start 132.75 103.5) (end 134 104.75) (width 0.2) (layer "B.Cu") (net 19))
 (segment (start 147.171735 103.951) (end 152.7 98.422735) (width 0.2) (layer "B.Cu") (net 19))
 (segment (start 152.737 96.003) (end 155.24 93.5) (width 0.2) (layer "F.Cu") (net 4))
 (segment (start 145 96.003) (end 152.737 96.003) (width 0.2) (layer "F.Cu") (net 4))
 (via (at 145 96.003) (size 0.6) (drill 0.3) (layers "F.Cu" "B.Cu") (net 4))
 (segment (start 123.2155 102.8303) (end 123.2155 94.862593) (width 0.2) (layer "B.Cu") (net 4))
 (segment (start 123.800993 94.2771) (end 124.629007 94.2771) (width 0.2) (layer "B.Cu") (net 4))
 (segment (start 124.629007 94.2771) (end 126.354907 96.003) (width 0.2) (layer "B.Cu") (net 4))
 (segment (start 123.2155 94.862593) (end 123.800993 94.2771) (width 0.2) (layer "B.Cu") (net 4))
 (segment (start 124.215 103.8298) (end 123.2155 102.8303) (width 0.2) (layer "B.Cu") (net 4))
 (segment (start 126.354907 96.003) (end 145 96.003) (width 0.2) (layer "B.Cu") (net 4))
 (segment (start 143.1736 108.1064) (end 157.78 93.5) (width 0.2) (layer "F.Cu") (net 20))
 (segment (start 124.215 108.1064) (end 143.1736 108.1064) (width 0.2) (layer "F.Cu") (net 20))
 (segment (start 141.2261 93.16905) (end 137.55705 89.5) (width 0.2) (layer "F.Cu") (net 33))
 (segment (start 132 96.88) (end 133.011 97.891) (width 0.2) (layer "F.Cu") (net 33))
 (segment (start 133.011 97.891) (end 141.6161 97.891) (width 0.2) (layer "F.Cu") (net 33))
 (segment (start 141.6161 97.891) (end 141.851 97.6561) (width 0.2) (layer "F.Cu") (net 33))
 (segment (start 141.851 97.6561) (end 141.851 96.478265) (width 0.2) (layer "F.Cu") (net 33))
 (segment (start 141.2261 95.853365) (end 141.2261 93.16905) (width 0.2) (layer "F.Cu") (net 33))
 (segment (start 141.851 96.478265) (end 141.2261 95.853365) (width 0.2) (layer "F.Cu") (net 33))
 (segment (start 137.55705 89.5) (end 137.5 89.5) (width 0.2) (layer "F.Cu") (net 33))
 (via (at 137.5 89.5) (size 0.6) (drill 0.3) (layers "F.Cu" "B.Cu") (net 33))
 (segment (start 132 112.12) (end 132 96.88) (width 0.2) (layer "B.Cu") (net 33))
 (segment (start 137.5 89.5) (end 137.46 89.46) (width 0.2) (layer "B.Cu") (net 33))
 (segment (start 137.46 89.46) (end 137.46 78.26) (width 0.2) (layer "B.Cu") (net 33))
 (segment (start 127.2304 98.292) (end 141.7822 98.292) (width 0.2) (layer "F.Cu") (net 13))
 (segment (start 144.8242 95.25) (end 148.41 95.25) (width 0.2) (layer "F.Cu") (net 13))
 (segment (start 148.41 95.25) (end 150.16 93.5) (width 0.2) (layer "F.Cu") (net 13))
 (segment (start 124.215 95.2766) (end 127.2304 98.292) (width 0.2) (layer "F.Cu") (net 13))
 (segment (start 141.7822 98.292) (end 144.8242 95.25) (width 0.2) (layer "F.Cu") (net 13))
 (segment (start 158.23605 77.159) (end 151.261 77.159) (width 0.2) (layer "B.Cu") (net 5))
 (segment (start 161.75 113) (end 160.5 113) (width 0.2) (layer "B.Cu") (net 5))
 (segment (start 160.049 98.114265) (end 158.881 96.946265) (width 0.2) (layer "B.Cu") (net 5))
 (segment (start 158.881 77.80395) (end 158.23605 77.159) (width 0.2) (layer "B.Cu") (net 5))
 (segment (start 151.261 77.159) (end 150.16 78.26) (width 0.2) (layer "B.Cu") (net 5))
 (segment (start 160.049 112.549) (end 160.049 98.114265) (width 0.2) (layer "B.Cu") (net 5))
 (segment (start 160.5 113) (end 160.049 112.549) (width 0.2) (layer "B.Cu") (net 5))
 (segment (start 158.881 96.946265) (end 158.881 77.80395) (width 0.2) (layer "B.Cu") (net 5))
 (segment (start 137.08 96.88) (end 136.443604 96.88) (width 0.2) (layer "F.Cu") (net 1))
 (segment (start 136.443604 96.88) (end 133.5 93.936396) (width 0.2) (layer "F.Cu") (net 1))
 (segment (start 133.5 93.936396) (end 133.5 93.06295) (width 0.2) (layer "F.Cu") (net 1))
 (segment (start 118.0611 83.4463) (end 112.785 78.1702) (width 0.2) (layer "F.Cu") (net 1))
 (segment (start 123.88335 83.4463) (end 118.0611 83.4463) (width 0.2) (layer "F.Cu") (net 1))
 (segment (start 133.5 93.06295) (end 123.88335 83.4463) (width 0.2) (layer "F.Cu") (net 1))
 (segment (start 134.54 96.88) (end 132.261 94.601) (width 0.2) (layer "F.Cu") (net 35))
 (segment (start 126.601 91.972493) (end 118.475807 83.8473) (width 0.2) (layer "F.Cu") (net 35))
 (segment (start 132.261 94.601) (end 126.601 94.601) (width 0.2) (layer "F.Cu") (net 35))
 (segment (start 114.1855 83.8473) (end 112.785 82.4468) (width 0.2) (layer "F.Cu") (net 35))
 (segment (start 126.601 94.601) (end 126.601 91.972493) (width 0.2) (layer "F.Cu") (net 35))
 (segment (start 118.475807 83.8473) (end 114.1855 83.8473) (width 0.2) (layer "F.Cu") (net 35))
 (segment (start 129.46 96.88) (end 128.123496 96.88) (width 0.2) (layer "F.Cu") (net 7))
 (segment (start 128.123496 96.88) (end 117.966896 86.7234) (width 0.2) (layer "F.Cu") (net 7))
 (segment (start 117.966896 86.7234) (end 112.785 86.7234) (width 0.2) (layer "F.Cu") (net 7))
 (segment (start 126.92 96.88) (end 126.92 96.243604) (width 0.2) (layer "F.Cu") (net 36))
 (segment (start 121.676396 91) (end 112.785 91) (width 0.2) (layer "F.Cu") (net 36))
 (segment (start 126.92 96.243604) (end 121.676396 91) (width 0.2) (layer "F.Cu") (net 36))
 (segment (start 123.2155 105.7071) (end 123.2155 109.051896) (width 0.2) (layer "F.Cu") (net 12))
 (segment (start 112.785 95.2766) (end 123.2155 105.7071) (width 0.2) (layer "F.Cu") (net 12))
 (segment (start 123.2155 109.051896) (end 126.283604 112.12) (width 0.2) (layer "F.Cu") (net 12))
 (segment (start 126.283604 112.12) (end 126.92 112.12) (width 0.2) (layer "F.Cu") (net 12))
 (segment (start 126.1028 112.871) (end 128.709 112.871) (width 0.2) (layer "F.Cu") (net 37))
 (segment (start 128.709 112.871) (end 129.46 112.12) (width 0.2) (layer "F.Cu") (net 37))
 (segment (start 112.785 99.5532) (end 126.1028 112.871) (width 0.2) (layer "F.Cu") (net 37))
 (segment (start 122.2272 113.272) (end 133.388 113.272) (width 0.2) (layer "F.Cu") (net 3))
 (segment (start 112.785 103.8298) (end 122.2272 113.272) (width 0.2) (layer "F.Cu") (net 3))
 (segment (start 133.388 113.272) (end 134.54 112.12) (width 0.2) (layer "F.Cu") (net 3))
 (segment (start 135.527 113.673) (end 137.08 112.12) (width 0.2) (layer "F.Cu") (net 38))
 (segment (start 112.785 108.1064) (end 118.3516 113.673) (width 0.2) (layer "F.Cu") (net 38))
 (segment (start 118.3516 113.673) (end 135.527 113.673) (width 0.2) (layer "F.Cu") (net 38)))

